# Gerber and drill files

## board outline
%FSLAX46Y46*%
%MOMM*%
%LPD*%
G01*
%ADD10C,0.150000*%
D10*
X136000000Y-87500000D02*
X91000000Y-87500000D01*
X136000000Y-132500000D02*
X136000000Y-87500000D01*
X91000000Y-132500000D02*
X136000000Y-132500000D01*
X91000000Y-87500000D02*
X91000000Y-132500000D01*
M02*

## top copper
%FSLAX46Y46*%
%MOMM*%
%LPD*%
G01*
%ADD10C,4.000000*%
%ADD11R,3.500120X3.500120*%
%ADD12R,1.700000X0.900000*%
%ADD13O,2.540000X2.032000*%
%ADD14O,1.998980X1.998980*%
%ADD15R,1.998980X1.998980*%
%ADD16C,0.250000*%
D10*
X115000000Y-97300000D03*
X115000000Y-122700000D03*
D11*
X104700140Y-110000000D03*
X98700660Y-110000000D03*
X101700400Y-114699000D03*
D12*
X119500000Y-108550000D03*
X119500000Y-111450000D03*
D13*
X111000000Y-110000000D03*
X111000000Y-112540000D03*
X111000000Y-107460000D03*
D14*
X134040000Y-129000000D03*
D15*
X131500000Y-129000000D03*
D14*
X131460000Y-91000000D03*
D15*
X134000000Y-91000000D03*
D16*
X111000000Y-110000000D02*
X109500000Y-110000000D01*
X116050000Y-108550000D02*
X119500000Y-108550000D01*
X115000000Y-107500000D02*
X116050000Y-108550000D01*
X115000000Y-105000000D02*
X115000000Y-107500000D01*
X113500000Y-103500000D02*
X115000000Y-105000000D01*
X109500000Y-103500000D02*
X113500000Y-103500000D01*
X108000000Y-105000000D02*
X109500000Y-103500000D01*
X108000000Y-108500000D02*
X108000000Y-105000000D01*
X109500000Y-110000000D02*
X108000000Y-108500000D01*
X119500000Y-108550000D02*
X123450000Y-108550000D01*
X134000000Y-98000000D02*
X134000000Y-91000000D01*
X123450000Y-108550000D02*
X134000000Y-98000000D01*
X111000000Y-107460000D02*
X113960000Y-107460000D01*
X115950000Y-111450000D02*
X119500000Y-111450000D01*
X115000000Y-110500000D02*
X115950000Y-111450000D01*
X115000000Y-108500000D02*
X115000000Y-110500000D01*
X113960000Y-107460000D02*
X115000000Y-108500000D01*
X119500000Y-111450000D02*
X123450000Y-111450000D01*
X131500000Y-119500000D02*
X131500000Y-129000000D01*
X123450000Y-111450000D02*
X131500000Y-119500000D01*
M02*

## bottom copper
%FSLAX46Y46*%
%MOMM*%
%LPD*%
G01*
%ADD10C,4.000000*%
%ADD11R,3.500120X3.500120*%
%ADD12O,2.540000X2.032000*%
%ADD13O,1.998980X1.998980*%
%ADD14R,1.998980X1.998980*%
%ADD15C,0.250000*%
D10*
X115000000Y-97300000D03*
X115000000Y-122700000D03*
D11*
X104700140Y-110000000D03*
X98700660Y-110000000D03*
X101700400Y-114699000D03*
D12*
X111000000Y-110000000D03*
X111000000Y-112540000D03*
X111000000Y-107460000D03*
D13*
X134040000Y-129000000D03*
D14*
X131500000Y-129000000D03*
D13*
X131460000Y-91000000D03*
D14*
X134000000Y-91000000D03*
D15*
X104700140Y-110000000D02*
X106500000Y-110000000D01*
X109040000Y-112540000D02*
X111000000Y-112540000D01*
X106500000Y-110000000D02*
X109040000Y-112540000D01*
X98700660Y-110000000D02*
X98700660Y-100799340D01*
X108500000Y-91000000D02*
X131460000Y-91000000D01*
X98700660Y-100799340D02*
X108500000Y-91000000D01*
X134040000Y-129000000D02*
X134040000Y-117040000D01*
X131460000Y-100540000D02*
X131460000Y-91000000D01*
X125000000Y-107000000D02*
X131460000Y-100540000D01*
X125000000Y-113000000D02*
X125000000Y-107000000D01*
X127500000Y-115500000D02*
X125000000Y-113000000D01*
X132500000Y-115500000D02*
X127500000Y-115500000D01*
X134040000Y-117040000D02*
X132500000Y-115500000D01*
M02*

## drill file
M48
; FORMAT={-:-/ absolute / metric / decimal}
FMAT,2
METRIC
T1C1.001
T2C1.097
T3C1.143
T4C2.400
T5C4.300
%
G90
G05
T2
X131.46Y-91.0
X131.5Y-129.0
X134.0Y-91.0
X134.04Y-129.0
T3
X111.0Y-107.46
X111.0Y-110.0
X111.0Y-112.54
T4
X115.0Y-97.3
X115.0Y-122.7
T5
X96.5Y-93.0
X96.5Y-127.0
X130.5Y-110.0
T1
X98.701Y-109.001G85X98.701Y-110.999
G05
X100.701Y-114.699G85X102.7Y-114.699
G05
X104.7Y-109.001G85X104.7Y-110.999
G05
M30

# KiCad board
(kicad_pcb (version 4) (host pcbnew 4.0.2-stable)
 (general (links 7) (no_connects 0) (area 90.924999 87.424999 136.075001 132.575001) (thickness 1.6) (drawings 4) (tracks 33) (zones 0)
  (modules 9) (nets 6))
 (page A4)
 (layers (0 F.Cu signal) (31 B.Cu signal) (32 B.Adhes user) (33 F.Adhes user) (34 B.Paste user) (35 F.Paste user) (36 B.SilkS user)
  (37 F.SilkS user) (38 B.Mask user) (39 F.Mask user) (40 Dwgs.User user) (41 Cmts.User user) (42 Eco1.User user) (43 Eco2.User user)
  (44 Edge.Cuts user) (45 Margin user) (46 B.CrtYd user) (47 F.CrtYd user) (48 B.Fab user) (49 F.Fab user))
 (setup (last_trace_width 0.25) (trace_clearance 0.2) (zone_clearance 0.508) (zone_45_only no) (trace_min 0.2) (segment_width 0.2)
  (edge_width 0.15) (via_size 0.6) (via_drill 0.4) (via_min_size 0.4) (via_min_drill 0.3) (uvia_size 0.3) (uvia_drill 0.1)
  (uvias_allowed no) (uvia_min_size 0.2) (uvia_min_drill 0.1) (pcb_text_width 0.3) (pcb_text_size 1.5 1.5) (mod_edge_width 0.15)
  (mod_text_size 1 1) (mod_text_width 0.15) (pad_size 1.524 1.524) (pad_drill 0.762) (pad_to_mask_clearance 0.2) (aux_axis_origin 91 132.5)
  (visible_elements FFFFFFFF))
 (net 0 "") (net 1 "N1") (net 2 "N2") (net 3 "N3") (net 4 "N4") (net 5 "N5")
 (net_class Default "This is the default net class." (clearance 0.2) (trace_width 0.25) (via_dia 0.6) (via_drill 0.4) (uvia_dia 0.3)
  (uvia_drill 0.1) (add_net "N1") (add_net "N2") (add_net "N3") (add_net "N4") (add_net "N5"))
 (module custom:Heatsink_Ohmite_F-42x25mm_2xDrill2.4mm (layer F.Cu) (at 115 110 270)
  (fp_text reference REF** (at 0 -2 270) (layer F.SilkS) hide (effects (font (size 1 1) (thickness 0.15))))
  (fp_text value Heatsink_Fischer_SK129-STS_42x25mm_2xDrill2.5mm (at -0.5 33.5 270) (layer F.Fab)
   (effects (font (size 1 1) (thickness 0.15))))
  (pad 1 thru_hole circle (at -12.7 0 270) (size 4 4) (drill 2.4) (layers *.Cu *.Mask F.SilkS))
  (pad 1 thru_hole circle (at 12.7 0 270) (size 4 4) (drill 2.4) (layers *.Cu *.Mask F.SilkS)))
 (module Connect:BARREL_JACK (layer F.Cu) (at 98.5 110)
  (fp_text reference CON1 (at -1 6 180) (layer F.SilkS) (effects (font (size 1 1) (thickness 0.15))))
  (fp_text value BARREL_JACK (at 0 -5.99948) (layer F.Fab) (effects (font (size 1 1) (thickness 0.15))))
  (pad 1 thru_hole rect (at 6.20014 0) (size 3.50012 3.50012) (drill oval 1.00076 2.99974) (layers *.Cu *.Mask F.SilkS) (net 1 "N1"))
  (pad 2 thru_hole rect (at 0.20066 0) (size 3.50012 3.50012) (drill oval 1.00076 2.99974) (layers *.Cu *.Mask F.SilkS) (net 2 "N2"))
  (pad 3 thru_hole rect (at 3.2004 4.699) (size 3.50012 3.50012) (drill oval 2.99974 1.00076) (layers *.Cu *.Mask F.SilkS) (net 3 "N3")))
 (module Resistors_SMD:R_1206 (layer F.Cu) (at 119.5 110 270)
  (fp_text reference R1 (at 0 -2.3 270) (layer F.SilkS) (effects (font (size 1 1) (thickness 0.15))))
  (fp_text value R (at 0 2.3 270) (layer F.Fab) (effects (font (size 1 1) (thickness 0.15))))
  (pad 1 smd rect (at -1.45 0 270) (size 0.9 1.7) (layers F.Cu F.Paste F.Mask) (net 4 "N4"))
  (pad 2 smd rect (at 1.45 0 270) (size 0.9 1.7) (layers F.Cu F.Paste F.Mask) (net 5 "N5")))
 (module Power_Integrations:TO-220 (layer F.Cu) (at 111 110 270)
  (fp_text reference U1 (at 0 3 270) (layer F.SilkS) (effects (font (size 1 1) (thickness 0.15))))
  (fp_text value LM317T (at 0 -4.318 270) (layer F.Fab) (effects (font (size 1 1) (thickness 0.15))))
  (pad 2 thru_hole oval (at 0 0 270) (size 2.032 2.54) (drill 1.143) (layers *.Cu *.Mask F.SilkS) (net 4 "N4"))
  (pad 3 thru_hole oval (at 2.54 0 270) (size 2.032 2.54) (drill 1.143) (layers *.Cu *.Mask F.SilkS) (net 1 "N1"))
  (pad 1 thru_hole oval (at -2.54 0 270) (size 2.032 2.54) (drill 1.143) (layers *.Cu *.Mask F.SilkS) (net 5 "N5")))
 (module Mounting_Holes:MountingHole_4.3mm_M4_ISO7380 (layer F.Cu) (at 96.5 93)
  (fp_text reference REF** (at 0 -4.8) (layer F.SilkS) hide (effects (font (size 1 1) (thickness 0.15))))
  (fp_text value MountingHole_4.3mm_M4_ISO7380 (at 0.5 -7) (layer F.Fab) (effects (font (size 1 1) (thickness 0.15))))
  (pad 1 np_thru_hole circle (at 0 0) (size 4.3 4.3) (drill 4.3) (layers *.Cu *.Mask F.SilkS)))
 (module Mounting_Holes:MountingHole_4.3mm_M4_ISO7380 (layer F.Cu) (at 96.5 127)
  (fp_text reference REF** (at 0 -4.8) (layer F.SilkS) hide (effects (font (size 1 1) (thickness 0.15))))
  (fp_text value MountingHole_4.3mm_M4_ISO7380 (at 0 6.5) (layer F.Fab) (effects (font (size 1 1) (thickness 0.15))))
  (pad 1 np_thru_hole circle (at 0 0) (size 4.3 4.3) (drill 4.3) (layers *.Cu *.Mask F.SilkS)))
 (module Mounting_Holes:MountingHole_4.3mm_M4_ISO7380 (layer F.Cu) (at 130.5 110)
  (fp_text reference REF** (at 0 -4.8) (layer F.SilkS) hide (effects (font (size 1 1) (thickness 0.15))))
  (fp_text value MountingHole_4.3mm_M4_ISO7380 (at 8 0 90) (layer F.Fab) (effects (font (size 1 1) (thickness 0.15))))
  (pad 1 np_thru_hole circle (at 0 0) (size 4.3 4.3) (drill 4.3) (layers *.Cu *.Mask F.SilkS)))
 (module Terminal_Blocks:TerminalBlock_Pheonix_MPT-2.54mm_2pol (layer F.Cu) (at 131.5 129)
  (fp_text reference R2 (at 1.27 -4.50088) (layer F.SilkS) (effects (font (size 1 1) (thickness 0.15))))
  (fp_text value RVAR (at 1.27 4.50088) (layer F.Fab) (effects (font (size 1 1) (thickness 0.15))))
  (pad 2 thru_hole oval (at 2.54 0) (size 1.99898 1.99898) (drill 1.09728) (layers *.Cu *.Mask F.SilkS) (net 2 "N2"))
  (pad 1 thru_hole rect (at 0 0) (size 1.99898 1.99898) (drill 1.09728) (layers *.Cu *.Mask F.SilkS) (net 5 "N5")))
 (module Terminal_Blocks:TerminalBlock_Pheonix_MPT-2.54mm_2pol (layer F.Cu) (at 134 91 180)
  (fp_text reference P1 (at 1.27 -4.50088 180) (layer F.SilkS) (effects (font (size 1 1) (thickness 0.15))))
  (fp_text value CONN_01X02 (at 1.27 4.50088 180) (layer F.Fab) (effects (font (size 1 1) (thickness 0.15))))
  (pad 2 thru_hole oval (at 2.54 0 180) (size 1.99898 1.99898) (drill 1.09728) (layers *.Cu *.Mask F.SilkS) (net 2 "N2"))
  (pad 1 thru_hole rect (at 0 0 180) (size 1.99898 1.99898) (drill 1.09728) (layers *.Cu *.Mask F.SilkS) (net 4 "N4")))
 (gr_line (start 136 87.5) (end 91 87.5) (angle 90) (layer Edge.Cuts) (width 0.15))
 (gr_line (start 136 132.5) (end 136 87.5) (angle 90) (layer Edge.Cuts) (width 0.15))
 (gr_line (start 91 132.5) (end 136 132.5) (angle 90) (layer Edge.Cuts) (width 0.15))
 (gr_line (start 91 87.5) (end 91 132.5) (angle 90) (layer Edge.Cuts) (width 0.15))
 (segment (start 104.70014 110) (end 106.5 110) (width 0.25) (layer B.Cu) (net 1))
 (segment (start 109.04 112.54) (end 111 112.54) (width 0.25) (layer B.Cu) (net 1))
 (segment (start 106.5 110) (end 109.04 112.54) (width 0.25) (layer B.Cu) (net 1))
 (segment (start 98.70066 110) (end 98.70066 100.79934) (width 0.25) (layer B.Cu) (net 2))
 (segment (start 108.5 91) (end 131.46 91) (width 0.25) (layer B.Cu) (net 2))
 (segment (start 98.70066 100.79934) (end 108.5 91) (width 0.25) (layer B.Cu) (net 2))
 (segment (start 134.04 129) (end 134.04 117.04) (width 0.25) (layer B.Cu) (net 2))
 (segment (start 131.46 100.54) (end 131.46 91) (width 0.25) (layer B.Cu) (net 2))
 (segment (start 125 107) (end 131.46 100.54) (width 0.25) (layer B.Cu) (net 2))
 (segment (start 125 113) (end 125 107) (width 0.25) (layer B.Cu) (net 2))
 (segment (start 127.5 115.5) (end 125 113) (width 0.25) (layer B.Cu) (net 2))
 (segment (start 132.5 115.5) (end 127.5 115.5) (width 0.25) (layer B.Cu) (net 2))
 (segment (start 134.04 117.04) (end 132.5 115.5) (width 0.25) (layer B.Cu) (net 2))
 (segment (start 111 110) (end 109.5 110) (width 0.25) (layer F.Cu) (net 4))
 (segment (start 116.05 108.55) (end 119.5 108.55) (width 0.25) (layer F.Cu) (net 4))
 (segment (start 115 107.5) (end 116.05 108.55) (width 0.25) (layer F.Cu) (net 4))
 (segment (start 115 105) (end 115 107.5) (width 0.25) (layer F.Cu) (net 4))
 (segment (start 113.5 103.5) (end 115 105) (width 0.25) (layer F.Cu) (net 4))
 (segment (start 109.5 103.5) (end 113.5 103.5) (width 0.25) (layer F.Cu) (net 4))
 (segment (start 108 105) (end 109.5 103.5) (width 0.25) (layer F.Cu) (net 4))
 (segment (start 108 108.5) (end 108 105) (width 0.25) (layer F.Cu) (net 4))
 (segment (start 109.5 110) (end 108 108.5) (width 0.25) (layer F.Cu) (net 4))
 (segment (start 119.5 108.55) (end 123.45 108.55) (width 0.25) (layer F.Cu) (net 4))
 (segment (start 134 98) (end 134 91) (width 0.25) (layer F.Cu) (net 4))
 (segment (start 123.45 108.55) (end 134 98) (width 0.25) (layer F.Cu) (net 4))
 (segment (start 111 107.46) (end 113.96 107.46) (width 0.25) (layer F.Cu) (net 5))
 (segment (start 115.95 111.45) (end 119.5 111.45) (width 0.25) (layer F.Cu) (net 5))
 (segment (start 115 110.5) (end 115.95 111.45) (width 0.25) (layer F.Cu) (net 5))
 (segment (start 115 108.5) (end 115 110.5) (width 0.25) (layer F.Cu) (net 5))
 (segment (start 113.96 107.46) (end 115 108.5) (width 0.25) (layer F.Cu) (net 5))
 (segment (start 119.5 111.45) (end 123.45 111.45) (width 0.25) (layer F.Cu) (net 5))
 (segment (start 131.5 119.5) (end 131.5 129) (width 0.25) (layer F.Cu) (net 5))
 (segment (start 123.45 111.45) (end 131.5 119.5) (width 0.25) (layer F.Cu) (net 5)))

